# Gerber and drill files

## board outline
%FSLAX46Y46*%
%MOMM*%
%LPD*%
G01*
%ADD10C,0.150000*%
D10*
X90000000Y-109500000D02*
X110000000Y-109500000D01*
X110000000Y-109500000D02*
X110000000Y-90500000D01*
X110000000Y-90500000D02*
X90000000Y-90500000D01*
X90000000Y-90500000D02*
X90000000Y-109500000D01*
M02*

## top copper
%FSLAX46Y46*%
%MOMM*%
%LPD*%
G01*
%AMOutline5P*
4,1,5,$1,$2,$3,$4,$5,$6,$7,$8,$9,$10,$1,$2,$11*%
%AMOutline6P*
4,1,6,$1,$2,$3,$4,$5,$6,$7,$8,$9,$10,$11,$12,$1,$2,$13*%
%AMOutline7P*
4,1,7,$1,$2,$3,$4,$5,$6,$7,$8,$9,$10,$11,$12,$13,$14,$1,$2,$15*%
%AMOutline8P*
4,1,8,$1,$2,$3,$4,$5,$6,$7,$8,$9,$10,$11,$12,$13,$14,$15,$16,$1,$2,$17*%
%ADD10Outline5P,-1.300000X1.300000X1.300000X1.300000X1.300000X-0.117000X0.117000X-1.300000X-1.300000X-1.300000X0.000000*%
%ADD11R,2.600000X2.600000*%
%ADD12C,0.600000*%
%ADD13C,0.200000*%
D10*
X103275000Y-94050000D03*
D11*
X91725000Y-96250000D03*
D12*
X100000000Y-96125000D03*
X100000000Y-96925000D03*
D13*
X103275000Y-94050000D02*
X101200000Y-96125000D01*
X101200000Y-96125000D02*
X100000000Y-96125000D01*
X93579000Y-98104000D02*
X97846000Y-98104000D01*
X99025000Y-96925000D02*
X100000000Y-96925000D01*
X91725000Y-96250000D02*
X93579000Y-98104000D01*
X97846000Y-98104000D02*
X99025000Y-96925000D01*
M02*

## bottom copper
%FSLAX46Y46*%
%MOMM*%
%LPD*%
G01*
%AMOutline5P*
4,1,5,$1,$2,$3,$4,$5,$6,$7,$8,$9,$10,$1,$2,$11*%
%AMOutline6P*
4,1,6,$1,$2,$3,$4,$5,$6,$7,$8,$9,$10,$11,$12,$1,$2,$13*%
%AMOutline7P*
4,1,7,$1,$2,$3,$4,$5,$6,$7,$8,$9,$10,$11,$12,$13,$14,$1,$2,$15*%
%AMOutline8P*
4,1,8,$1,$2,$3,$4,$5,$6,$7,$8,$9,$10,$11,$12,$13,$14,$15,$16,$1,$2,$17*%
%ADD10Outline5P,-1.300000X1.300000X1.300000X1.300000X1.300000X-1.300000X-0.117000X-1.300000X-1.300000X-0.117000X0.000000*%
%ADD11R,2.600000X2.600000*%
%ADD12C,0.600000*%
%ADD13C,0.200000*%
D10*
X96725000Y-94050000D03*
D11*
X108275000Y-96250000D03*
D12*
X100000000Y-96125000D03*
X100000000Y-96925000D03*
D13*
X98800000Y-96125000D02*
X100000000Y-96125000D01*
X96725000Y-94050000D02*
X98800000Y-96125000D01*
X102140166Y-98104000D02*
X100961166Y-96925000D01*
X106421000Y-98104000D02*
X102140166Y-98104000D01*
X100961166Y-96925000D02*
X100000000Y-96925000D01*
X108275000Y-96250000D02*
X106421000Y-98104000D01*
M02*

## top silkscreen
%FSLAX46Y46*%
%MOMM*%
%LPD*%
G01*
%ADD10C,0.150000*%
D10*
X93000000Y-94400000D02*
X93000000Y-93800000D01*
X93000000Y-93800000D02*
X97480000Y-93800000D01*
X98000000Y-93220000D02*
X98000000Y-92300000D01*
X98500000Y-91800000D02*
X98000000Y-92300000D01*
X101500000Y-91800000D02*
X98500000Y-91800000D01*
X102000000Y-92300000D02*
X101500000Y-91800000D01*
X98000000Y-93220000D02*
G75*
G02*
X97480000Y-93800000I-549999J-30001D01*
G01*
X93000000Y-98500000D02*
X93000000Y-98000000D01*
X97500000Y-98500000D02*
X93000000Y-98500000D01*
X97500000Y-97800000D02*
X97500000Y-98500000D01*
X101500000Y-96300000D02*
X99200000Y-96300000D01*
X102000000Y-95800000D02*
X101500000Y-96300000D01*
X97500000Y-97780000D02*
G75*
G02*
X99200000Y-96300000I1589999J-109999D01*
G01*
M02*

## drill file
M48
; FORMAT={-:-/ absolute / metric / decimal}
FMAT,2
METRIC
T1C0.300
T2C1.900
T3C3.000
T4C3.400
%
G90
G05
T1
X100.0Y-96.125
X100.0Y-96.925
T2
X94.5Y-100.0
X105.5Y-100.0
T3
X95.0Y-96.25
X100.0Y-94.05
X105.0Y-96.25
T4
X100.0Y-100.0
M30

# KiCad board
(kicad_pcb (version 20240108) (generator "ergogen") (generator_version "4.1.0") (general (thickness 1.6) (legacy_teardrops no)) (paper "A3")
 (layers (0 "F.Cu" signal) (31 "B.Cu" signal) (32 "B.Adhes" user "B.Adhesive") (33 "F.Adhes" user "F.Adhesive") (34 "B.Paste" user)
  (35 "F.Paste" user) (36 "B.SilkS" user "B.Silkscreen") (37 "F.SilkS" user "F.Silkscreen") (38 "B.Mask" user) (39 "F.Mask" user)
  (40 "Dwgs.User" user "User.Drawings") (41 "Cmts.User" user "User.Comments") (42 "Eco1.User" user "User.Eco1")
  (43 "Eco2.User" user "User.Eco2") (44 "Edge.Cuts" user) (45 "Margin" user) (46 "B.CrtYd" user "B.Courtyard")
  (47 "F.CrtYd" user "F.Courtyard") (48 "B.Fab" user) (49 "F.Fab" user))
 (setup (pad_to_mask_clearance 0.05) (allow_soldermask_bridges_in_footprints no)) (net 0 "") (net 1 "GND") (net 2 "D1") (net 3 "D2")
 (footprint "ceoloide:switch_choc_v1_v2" (layer "B.Cu") (at 100 100 0)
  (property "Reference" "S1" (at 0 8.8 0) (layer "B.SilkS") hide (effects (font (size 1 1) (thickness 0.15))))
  (pad "" np_thru_hole circle (at 0 0 0) (size 3.4 3.4) (drill 3.4) (layers "*.Cu" "*.Mask"))
  (pad "" np_thru_hole circle (at 5.5 0 0) (size 1.9 1.9) (drill 1.9) (layers "*.Cu" "*.Mask"))
  (pad "" np_thru_hole circle (at -5.5 0 0) (size 1.9 1.9) (drill 1.9) (layers "*.Cu" "*.Mask"))
  (pad "" np_thru_hole circle (at 0 -5.95 0) (size 3 3) (drill 3) (layers "*.Cu" "*.Mask"))
  (fp_line (start -7 -5.6) (end -7 -6.2) (layer "F.SilkS") (stroke (width 0.15) (type solid)))
  (fp_line (start -7 -6.2) (end -2.52 -6.2) (layer "F.SilkS") (stroke (width 0.15) (type solid)))
  (fp_line (start -2 -6.78) (end -2 -7.7) (layer "F.SilkS") (stroke (width 0.15) (type solid)))
  (fp_line (start -1.5 -8.2) (end -2 -7.7) (layer "F.SilkS") (stroke (width 0.15) (type solid)))
  (fp_line (start 1.5 -8.2) (end -1.5 -8.2) (layer "F.SilkS") (stroke (width 0.15) (type solid)))
  (fp_line (start 2 -7.7) (end 1.5 -8.2) (layer "F.SilkS") (stroke (width 0.15) (type solid)))
  (fp_arc (start -2 -6.78) (mid -2.139878 -6.382304) (end -2.52 -6.2) (layer "F.SilkS") (stroke (width 0.15) (type solid)))
  (fp_line (start -7 -1.5) (end -7 -2) (layer "F.SilkS") (stroke (width 0.15) (type solid)))
  (fp_line (start -2.5 -1.5) (end -7 -1.5) (layer "F.SilkS") (stroke (width 0.15) (type solid)))
  (fp_line (start -2.5 -2.2) (end -2.5 -1.5) (layer "F.SilkS") (stroke (width 0.15) (type solid)))
  (fp_line (start 1.5 -3.7) (end -0.8 -3.7) (layer "F.SilkS") (stroke (width 0.15) (type solid)))
  (fp_line (start 2 -4.2) (end 1.5 -3.7) (layer "F.SilkS") (stroke (width 0.15) (type solid)))
  (fp_arc (start -2.5 -2.22) (mid -1.956518 -3.312082) (end -0.8 -3.7) (layer "F.SilkS") (stroke (width 0.15) (type solid)))
  (pad "" np_thru_hole circle (at -5 -3.75 195) (size 3 3) (drill 3) (layers "*.Cu" "*.Mask"))
  (pad "1" smd roundrect (at 3.275 -5.95 0) (size 2.6 2.6) (layers "F.Cu" "F.Paste" "F.Mask") (roundrect_rratio 0) (chamfer_ratio 0.455)
   (chamfer bottom_right) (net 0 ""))
  (pad "2" smd rect (at -8.275 -3.75 0) (size 2.6 2.6) (layers "F.Cu" "F.Paste" "F.Mask") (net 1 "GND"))
  (pad "1" smd roundrect (at -3.275 -5.95 0) (size 2.6 2.6) (layers "B.Cu" "B.Paste" "B.Mask") (roundrect_rratio 0) (chamfer_ratio 0.455)
   (chamfer bottom_left) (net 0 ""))
  (pad "2" smd rect (at 8.275 -3.75 0) (size 2.6 2.6) (layers "B.Cu" "B.Paste" "B.Mask") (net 1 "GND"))
  (pad "" np_thru_hole circle (at 5 -3.75 195) (size 3 3) (drill 3) (layers "*.Cu" "*.Mask")))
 (segment (start 103.275 94.05) (end 101.2 96.125) (width 0.2) (layer "F.Cu") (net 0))
 (segment (start 101.2 96.125) (end 100 96.125) (width 0.2) (layer "F.Cu") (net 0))
 (via (at 100 96.125) (size 0.6) (drill 0.3) (layers "F.Cu" "B.Cu") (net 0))
 (segment (start 98.8 96.125) (end 100 96.125) (width 0.2) (layer "B.Cu") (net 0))
 (segment (start 96.725 94.05) (end 98.8 96.125) (width 0.2) (layer "B.Cu") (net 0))
 (segment (start 93.579 98.104) (end 97.846 98.104) (width 0.2) (layer "F.Cu") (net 1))
 (segment (start 99.025 96.925) (end 100 96.925) (width 0.2) (layer "F.Cu") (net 1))
 (segment (start 91.725 96.25) (end 93.579 98.104) (width 0.2) (layer "F.Cu") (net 1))
 (segment (start 97.846 98.104) (end 99.025 96.925) (width 0.2) (layer "F.Cu") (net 1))
 (via (at 100 96.925) (size 0.6) (drill 0.3) (layers "F.Cu" "B.Cu") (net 1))
 (segment (start 102.140166 98.104) (end 100.961166 96.925) (width 0.2) (layer "B.Cu") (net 1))
 (segment (start 106.421 98.104) (end 102.140166 98.104) (width 0.2) (layer "B.Cu") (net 1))
 (segment (start 100.961166 96.925) (end 100 96.925) (width 0.2) (layer "B.Cu") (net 1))
 (segment (start 108.275 96.25) (end 106.421 98.104) (width 0.2) (layer "B.Cu") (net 1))
 (gr_line (start 90 109.5) (end 110 109.5) (layer Edge.Cuts) (stroke (width 0.15) (type default)))
 (gr_line (start 110 109.5) (end 110 90.5) (layer Edge.Cuts) (stroke (width 0.15) (type default)))
 (gr_line (start 110 90.5) (end 90 90.5) (layer Edge.Cuts) (stroke (width 0.15) (type default)))
 (gr_line (start 90 90.5) (end 90 109.5) (layer Edge.Cuts) (stroke (width 0.15) (type default))))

